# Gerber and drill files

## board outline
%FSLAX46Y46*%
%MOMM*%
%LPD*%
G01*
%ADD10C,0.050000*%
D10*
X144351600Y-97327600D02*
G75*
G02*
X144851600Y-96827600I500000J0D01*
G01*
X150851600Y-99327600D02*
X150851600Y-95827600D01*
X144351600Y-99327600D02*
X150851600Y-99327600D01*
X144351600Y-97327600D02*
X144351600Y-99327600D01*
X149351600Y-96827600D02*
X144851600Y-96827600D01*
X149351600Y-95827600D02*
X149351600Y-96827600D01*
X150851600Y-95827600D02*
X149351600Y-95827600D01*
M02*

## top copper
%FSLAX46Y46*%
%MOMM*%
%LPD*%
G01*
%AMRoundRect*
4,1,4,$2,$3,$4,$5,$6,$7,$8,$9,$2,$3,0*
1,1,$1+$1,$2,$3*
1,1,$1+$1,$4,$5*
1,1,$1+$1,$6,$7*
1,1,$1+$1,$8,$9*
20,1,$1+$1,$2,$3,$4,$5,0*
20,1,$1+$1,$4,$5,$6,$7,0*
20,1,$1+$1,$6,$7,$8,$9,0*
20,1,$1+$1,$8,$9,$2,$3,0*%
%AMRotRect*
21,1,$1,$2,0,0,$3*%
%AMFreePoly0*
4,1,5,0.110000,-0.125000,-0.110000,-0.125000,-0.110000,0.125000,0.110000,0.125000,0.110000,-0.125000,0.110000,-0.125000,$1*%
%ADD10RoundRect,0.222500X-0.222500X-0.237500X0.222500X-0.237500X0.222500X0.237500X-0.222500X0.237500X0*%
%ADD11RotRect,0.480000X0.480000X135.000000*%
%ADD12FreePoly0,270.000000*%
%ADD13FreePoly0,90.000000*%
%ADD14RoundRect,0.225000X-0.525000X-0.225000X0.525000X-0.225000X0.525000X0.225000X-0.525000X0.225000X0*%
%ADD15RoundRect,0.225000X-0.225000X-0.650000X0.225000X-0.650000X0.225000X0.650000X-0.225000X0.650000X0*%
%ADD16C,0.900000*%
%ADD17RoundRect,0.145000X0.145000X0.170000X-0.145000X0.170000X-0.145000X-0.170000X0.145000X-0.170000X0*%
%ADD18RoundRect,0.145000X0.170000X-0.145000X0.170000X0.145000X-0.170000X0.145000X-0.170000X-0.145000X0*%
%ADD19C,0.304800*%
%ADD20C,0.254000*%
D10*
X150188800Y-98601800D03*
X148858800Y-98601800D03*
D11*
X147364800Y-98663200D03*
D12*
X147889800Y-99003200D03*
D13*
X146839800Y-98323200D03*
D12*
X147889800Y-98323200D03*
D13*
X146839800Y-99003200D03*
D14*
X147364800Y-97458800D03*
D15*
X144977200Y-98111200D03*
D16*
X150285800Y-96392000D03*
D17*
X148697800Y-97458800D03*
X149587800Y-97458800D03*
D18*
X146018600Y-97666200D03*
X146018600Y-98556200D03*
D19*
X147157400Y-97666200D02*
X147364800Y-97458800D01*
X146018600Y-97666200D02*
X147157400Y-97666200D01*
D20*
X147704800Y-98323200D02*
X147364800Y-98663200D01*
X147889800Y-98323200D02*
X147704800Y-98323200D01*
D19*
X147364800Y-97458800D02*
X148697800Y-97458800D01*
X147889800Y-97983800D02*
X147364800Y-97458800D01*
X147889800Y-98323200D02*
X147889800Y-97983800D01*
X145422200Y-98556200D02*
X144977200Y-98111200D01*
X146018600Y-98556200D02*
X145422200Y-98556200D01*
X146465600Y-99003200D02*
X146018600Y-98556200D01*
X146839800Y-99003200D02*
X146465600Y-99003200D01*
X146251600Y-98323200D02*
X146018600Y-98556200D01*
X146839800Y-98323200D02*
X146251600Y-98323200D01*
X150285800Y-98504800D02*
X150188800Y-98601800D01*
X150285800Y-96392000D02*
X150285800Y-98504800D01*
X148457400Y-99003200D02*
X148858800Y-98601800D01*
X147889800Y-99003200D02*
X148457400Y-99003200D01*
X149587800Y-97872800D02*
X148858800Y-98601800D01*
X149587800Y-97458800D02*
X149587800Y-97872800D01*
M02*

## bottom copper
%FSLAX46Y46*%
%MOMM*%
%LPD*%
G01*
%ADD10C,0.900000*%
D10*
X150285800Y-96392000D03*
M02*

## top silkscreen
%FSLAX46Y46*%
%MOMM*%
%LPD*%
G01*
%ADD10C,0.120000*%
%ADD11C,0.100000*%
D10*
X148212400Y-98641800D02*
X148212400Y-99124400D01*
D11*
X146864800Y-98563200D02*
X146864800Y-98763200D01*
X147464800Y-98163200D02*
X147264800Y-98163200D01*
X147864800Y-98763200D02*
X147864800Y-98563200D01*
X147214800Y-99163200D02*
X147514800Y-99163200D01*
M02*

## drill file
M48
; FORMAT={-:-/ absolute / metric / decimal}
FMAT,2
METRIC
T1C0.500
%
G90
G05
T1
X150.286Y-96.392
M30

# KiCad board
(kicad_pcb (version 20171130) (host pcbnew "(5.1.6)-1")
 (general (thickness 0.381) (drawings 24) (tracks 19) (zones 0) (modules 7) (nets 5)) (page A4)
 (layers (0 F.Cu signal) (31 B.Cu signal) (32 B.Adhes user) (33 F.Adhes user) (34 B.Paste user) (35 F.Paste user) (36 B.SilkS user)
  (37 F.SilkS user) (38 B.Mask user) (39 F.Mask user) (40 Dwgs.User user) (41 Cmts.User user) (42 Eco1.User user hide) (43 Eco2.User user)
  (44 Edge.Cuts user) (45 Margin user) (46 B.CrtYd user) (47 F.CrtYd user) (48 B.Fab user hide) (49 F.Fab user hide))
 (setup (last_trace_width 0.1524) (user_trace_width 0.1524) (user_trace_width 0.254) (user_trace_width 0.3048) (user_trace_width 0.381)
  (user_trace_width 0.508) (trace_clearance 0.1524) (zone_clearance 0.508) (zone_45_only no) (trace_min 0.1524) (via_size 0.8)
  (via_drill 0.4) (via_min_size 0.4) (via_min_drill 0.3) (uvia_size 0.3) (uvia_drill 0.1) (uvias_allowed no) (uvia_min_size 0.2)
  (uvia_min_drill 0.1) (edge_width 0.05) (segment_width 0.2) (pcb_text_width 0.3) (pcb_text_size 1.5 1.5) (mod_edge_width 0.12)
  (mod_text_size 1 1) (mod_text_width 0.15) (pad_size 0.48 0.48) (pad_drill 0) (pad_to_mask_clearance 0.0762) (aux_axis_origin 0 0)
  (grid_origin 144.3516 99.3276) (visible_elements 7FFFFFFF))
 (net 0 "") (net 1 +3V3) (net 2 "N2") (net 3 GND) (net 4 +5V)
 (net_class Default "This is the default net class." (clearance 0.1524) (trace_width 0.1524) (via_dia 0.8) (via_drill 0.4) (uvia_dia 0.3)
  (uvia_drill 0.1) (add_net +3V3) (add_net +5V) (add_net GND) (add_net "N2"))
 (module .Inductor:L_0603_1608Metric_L (layer F.Cu) (at 149.5238 98.6018)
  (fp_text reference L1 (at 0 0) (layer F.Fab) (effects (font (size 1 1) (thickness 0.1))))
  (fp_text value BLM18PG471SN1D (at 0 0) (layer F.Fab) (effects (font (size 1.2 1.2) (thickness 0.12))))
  (pad 2 smd roundrect (at 0.665 0) (size 0.89 0.92) (layers F.Cu F.Paste F.Mask) (roundrect_rratio 0.25) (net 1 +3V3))
  (pad 1 smd roundrect (at -0.665 0) (size 0.89 0.92) (layers F.Cu F.Paste F.Mask) (roundrect_rratio 0.25) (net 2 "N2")))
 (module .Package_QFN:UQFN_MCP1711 (layer F.Cu) (at 147.3648 98.6632 90)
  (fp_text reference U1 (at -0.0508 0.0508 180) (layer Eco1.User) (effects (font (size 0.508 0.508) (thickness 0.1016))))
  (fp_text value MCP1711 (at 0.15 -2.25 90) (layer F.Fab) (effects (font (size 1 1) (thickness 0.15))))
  (fp_line (start 0.1 -0.5) (end -0.1 -0.5) (layer F.SilkS) (width 0.1))
  (fp_line (start 0.5 0.1) (end 0.5 -0.1) (layer F.SilkS) (width 0.1))
  (fp_line (start -0.1 0.5) (end 0.1 0.5) (layer F.SilkS) (width 0.1))
  (fp_line (start -0.5 -0.15) (end -0.5 0.15) (layer F.SilkS) (width 0.1))
  (pad 5 smd rect (at 0 0 135) (size 0.48 0.48) (layers F.Cu F.Paste F.Mask) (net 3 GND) (solder_mask_margin 0.0254) (zone_connect 0))
  (pad 1 smd custom (at -0.34 0.525 270) (size 0.22 0.25) (layers F.Cu F.Paste F.Mask) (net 2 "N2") (zone_connect 0)
   (options (clearance outline) (anchor rect)) (primitives))
  (pad 3 smd custom (at 0.34 -0.525 90) (size 0.22 0.25) (layers F.Cu F.Paste F.Mask) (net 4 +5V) (zone_connect 0)
   (options (clearance outline) (anchor rect)) (primitives))
  (pad 2 smd custom (at 0.34 0.525 270) (size 0.22 0.25) (layers F.Cu F.Paste F.Mask) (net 3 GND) (zone_connect 0)
   (options (clearance outline) (anchor rect)) (primitives))
  (pad 4 smd custom (at -0.34 -0.525 90) (size 0.22 0.25) (layers F.Cu F.Paste F.Mask) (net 4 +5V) (zone_connect 0)
   (options (clearance outline) (anchor rect)) (primitives)))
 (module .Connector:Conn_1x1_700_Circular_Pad (layer F.Cu) (at 147.3648 97.4588)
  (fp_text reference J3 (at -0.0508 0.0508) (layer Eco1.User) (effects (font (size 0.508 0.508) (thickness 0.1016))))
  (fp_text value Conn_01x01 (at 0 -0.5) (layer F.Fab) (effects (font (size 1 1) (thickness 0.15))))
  (pad 1 smd roundrect (at 0 0) (size 1.5 0.9) (layers F.Cu F.Paste F.Mask) (roundrect_rratio 0.25) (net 3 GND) (solder_paste_margin -2)))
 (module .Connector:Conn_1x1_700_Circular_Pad (layer F.Cu) (at 144.9772 98.1112)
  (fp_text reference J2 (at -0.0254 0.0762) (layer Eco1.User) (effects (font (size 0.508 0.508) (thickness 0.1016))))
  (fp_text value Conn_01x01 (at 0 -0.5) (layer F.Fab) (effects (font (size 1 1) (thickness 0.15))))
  (pad 1 smd roundrect (at 0 0) (size 0.9 1.75) (layers F.Cu F.Paste F.Mask) (roundrect_rratio 0.25) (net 4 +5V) (solder_paste_margin -2)))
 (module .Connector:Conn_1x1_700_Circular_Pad (layer F.Cu) (at 150.2858 96.392)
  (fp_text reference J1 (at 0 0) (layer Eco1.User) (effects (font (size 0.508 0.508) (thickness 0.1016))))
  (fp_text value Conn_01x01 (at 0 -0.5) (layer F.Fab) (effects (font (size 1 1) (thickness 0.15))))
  (pad 1 thru_hole circle (at 0 0) (size 0.9 0.9) (drill 0.5) (layers *.Cu *.Mask) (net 1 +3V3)))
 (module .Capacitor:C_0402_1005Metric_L (layer F.Cu) (at 149.1428 97.4588 180)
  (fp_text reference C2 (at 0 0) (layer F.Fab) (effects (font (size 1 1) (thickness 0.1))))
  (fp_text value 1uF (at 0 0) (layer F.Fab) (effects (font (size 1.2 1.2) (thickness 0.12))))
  (pad 2 smd roundrect (at 0.445 0 180) (size 0.58 0.63) (layers F.Cu F.Paste F.Mask) (roundrect_rratio 0.25) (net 3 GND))
  (pad 1 smd roundrect (at -0.445 0 180) (size 0.58 0.63) (layers F.Cu F.Paste F.Mask) (roundrect_rratio 0.25) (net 2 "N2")))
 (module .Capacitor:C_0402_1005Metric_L (layer F.Cu) (at 146.0186 98.1112 90)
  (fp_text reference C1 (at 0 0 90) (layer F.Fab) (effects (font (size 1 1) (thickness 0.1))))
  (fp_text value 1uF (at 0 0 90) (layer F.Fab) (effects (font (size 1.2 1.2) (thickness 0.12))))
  (pad 2 smd roundrect (at 0.445 0 90) (size 0.58 0.63) (layers F.Cu F.Paste F.Mask) (roundrect_rratio 0.25) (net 3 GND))
  (pad 1 smd roundrect (at -0.445 0 90) (size 0.58 0.63) (layers F.Cu F.Paste F.Mask) (roundrect_rratio 0.25) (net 4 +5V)))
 (gr_line (start 148.2124 98.6418) (end 148.2124 99.1244) (layer F.SilkS) (width 0.12))
 (gr_arc (start 144.8516 97.3276) (end 144.8516 96.8276) (angle -90) (layer Edge.Cuts) (width 0.05))
 (gr_line (start 150.8516 99.3276) (end 150.8516 95.8276) (layer Edge.Cuts) (width 0.05))
 (gr_line (start 144.3516 99.3276) (end 150.8516 99.3276) (layer Edge.Cuts) (width 0.05))
 (gr_line (start 144.3516 97.3276) (end 144.3516 99.3276) (layer Edge.Cuts) (width 0.05))
 (gr_line (start 149.3516 96.8276) (end 144.8516 96.8276) (layer Edge.Cuts) (width 0.05))
 (gr_line (start 149.3516 95.8276) (end 149.3516 96.8276) (layer Edge.Cuts) (width 0.05))
 (gr_line (start 150.8516 95.8276) (end 149.3516 95.8276) (layer Edge.Cuts) (width 0.05))
 (segment (start 147.1574 97.6662) (end 147.3648 97.4588) (width 0.3048) (layer F.Cu) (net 3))
 (segment (start 146.0186 97.6662) (end 147.1574 97.6662) (width 0.3048) (layer F.Cu) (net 3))
 (segment (start 147.7048 98.3232) (end 147.3648 98.6632) (width 0.254) (layer F.Cu) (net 3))
 (segment (start 147.8898 98.3232) (end 147.7048 98.3232) (width 0.254) (layer F.Cu) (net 3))
 (segment (start 147.3648 97.4588) (end 148.6978 97.4588) (width 0.3048) (layer F.Cu) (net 3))
 (segment (start 147.8898 97.9838) (end 147.3648 97.4588) (width 0.3048) (layer F.Cu) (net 3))
 (segment (start 147.8898 98.3232) (end 147.8898 97.9838) (width 0.3048) (layer F.Cu) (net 3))
 (segment (start 145.4222 98.5562) (end 144.9772 98.1112) (width 0.3048) (layer F.Cu) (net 4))
 (segment (start 146.0186 98.5562) (end 145.4222 98.5562) (width 0.3048) (layer F.Cu) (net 4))
 (segment (start 146.4656 99.0032) (end 146.0186 98.5562) (width 0.3048) (layer F.Cu) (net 4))
 (segment (start 146.8398 99.0032) (end 146.4656 99.0032) (width 0.3048) (layer F.Cu) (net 4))
 (segment (start 146.2516 98.3232) (end 146.0186 98.5562) (width 0.3048) (layer F.Cu) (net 4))
 (segment (start 146.8398 98.3232) (end 146.2516 98.3232) (width 0.3048) (layer F.Cu) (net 4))
 (segment (start 150.2858 98.5048) (end 150.1888 98.6018) (width 0.3048) (layer F.Cu) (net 1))
 (segment (start 150.2858 96.392) (end 150.2858 98.5048) (width 0.3048) (layer F.Cu) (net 1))
 (segment (start 148.4574 99.0032) (end 148.8588 98.6018) (width 0.3048) (layer F.Cu) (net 2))
 (segment (start 147.8898 99.0032) (end 148.4574 99.0032) (width 0.3048) (layer F.Cu) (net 2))
 (segment (start 149.5878 97.8728) (end 148.8588 98.6018) (width 0.3048) (layer F.Cu) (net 2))
 (segment (start 149.5878 97.4588) (end 149.5878 97.8728) (width 0.3048) (layer F.Cu) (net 2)))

